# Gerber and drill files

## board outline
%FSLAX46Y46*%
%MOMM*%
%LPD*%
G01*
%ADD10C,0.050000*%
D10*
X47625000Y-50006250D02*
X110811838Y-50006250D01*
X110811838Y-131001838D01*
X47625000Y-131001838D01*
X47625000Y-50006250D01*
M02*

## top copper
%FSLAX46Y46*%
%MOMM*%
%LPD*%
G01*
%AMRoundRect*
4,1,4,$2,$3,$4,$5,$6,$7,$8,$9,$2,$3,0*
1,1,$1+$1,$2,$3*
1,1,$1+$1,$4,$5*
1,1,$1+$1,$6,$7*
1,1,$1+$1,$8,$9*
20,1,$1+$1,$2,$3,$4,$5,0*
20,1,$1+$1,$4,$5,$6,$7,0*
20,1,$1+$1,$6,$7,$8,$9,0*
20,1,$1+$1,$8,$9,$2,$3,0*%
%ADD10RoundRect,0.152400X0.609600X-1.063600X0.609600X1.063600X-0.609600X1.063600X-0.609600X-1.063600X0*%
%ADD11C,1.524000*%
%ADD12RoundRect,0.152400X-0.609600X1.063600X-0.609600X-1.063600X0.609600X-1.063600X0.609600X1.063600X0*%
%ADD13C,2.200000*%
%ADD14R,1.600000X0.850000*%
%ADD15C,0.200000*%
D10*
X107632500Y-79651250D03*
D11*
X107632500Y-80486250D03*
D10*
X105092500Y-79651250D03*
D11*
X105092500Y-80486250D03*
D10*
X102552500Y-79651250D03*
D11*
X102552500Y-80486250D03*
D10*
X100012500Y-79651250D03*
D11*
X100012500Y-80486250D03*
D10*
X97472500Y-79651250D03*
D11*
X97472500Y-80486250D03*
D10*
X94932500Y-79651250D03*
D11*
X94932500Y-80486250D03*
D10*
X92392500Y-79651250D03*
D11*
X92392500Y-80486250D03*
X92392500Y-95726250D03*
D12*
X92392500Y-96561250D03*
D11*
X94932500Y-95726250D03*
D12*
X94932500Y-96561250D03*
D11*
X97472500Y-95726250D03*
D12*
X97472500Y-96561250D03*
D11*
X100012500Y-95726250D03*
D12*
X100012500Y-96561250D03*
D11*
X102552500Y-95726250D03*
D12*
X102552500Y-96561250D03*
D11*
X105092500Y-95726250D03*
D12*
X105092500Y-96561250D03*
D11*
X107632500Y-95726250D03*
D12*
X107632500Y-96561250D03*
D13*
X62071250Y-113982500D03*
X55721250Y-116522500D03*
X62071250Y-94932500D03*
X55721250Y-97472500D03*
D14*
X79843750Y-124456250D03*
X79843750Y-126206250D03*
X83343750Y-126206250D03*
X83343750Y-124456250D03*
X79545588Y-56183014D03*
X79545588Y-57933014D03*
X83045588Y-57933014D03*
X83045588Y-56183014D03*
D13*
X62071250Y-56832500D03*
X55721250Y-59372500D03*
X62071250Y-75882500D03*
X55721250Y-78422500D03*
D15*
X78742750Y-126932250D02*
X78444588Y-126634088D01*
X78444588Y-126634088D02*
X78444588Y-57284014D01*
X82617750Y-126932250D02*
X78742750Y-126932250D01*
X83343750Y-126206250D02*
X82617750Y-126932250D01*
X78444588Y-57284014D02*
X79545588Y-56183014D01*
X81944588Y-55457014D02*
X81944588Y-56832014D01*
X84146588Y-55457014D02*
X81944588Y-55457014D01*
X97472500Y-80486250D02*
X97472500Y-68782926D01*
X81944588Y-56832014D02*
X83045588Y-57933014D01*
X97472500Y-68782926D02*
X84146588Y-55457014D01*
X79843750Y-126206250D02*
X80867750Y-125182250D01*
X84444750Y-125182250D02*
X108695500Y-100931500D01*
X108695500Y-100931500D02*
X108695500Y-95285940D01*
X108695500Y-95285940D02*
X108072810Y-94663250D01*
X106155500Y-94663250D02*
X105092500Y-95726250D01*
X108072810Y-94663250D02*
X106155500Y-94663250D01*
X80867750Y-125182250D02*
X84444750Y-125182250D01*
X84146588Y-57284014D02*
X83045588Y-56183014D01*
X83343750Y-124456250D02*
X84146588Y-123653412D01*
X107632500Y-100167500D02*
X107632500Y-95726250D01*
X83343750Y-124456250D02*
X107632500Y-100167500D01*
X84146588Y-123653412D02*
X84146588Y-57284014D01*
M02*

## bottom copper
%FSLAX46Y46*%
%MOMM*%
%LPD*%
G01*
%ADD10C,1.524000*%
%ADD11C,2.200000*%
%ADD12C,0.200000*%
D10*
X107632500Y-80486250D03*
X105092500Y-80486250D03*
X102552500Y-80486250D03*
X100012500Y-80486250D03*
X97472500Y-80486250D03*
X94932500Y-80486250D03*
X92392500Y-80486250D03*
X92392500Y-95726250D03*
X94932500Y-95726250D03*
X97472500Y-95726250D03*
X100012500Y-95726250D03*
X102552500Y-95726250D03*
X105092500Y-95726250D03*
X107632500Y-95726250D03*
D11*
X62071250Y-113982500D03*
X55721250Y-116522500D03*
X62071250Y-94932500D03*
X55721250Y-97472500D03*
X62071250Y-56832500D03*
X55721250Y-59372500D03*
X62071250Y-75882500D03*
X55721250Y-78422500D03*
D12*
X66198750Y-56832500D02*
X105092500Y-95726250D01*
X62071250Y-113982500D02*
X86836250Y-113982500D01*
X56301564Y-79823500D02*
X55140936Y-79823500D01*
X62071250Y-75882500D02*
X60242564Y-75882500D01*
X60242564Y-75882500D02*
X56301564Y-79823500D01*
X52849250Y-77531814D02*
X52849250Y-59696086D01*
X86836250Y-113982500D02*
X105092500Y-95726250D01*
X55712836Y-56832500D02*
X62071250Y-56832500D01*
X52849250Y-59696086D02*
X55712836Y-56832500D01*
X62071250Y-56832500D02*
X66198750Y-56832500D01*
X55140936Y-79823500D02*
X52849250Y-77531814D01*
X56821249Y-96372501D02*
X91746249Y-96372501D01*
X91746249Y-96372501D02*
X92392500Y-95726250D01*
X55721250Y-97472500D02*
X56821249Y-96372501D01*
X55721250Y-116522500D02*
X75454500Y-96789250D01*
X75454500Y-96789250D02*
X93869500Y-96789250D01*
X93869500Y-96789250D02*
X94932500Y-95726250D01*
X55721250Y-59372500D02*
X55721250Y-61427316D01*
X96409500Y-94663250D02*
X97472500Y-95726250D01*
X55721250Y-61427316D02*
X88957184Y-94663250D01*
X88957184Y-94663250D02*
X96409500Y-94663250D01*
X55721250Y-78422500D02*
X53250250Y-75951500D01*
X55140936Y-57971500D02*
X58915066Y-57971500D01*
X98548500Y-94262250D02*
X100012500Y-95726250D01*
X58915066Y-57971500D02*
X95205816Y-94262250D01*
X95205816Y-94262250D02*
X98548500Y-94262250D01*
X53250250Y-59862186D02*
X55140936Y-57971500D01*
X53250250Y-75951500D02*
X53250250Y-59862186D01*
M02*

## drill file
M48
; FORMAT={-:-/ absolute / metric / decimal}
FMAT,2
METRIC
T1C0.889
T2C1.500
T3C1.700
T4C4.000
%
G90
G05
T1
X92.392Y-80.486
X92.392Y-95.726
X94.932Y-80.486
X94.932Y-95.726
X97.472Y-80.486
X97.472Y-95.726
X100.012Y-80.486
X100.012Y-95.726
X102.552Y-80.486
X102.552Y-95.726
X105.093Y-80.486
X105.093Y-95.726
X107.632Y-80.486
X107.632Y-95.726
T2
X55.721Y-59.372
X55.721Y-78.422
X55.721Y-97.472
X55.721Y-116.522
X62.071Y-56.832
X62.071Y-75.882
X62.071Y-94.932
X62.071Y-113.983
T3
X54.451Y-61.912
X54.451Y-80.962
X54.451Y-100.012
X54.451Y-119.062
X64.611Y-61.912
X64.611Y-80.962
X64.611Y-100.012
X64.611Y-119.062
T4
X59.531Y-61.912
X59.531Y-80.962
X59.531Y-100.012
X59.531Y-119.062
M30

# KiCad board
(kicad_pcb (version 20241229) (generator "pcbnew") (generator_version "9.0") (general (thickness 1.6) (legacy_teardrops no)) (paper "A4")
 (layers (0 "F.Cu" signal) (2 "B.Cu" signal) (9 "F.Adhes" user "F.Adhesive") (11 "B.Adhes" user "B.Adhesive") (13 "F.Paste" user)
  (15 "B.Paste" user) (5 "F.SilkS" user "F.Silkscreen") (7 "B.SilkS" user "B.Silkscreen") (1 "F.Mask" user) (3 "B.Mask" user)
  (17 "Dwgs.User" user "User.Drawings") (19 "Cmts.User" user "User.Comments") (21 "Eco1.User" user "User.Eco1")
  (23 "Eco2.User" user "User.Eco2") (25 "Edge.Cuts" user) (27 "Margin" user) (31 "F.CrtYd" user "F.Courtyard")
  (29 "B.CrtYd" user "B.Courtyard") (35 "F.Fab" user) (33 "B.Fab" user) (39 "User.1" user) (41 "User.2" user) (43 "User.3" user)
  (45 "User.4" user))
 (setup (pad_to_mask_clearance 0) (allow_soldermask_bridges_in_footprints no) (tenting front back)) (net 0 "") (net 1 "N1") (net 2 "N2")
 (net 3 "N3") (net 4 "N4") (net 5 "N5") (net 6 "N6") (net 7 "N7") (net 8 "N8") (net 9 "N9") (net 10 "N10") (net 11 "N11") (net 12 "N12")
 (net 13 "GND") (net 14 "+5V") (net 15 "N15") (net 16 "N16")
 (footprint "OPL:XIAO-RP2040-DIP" (layer "F.Cu") (at 100.0125 88.10625 -90)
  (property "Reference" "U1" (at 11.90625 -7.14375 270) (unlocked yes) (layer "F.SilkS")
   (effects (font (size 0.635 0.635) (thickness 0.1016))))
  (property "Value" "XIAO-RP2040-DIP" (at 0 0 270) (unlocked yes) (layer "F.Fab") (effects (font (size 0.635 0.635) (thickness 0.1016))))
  (pad "1" smd roundrect (at -8.455 -7.62 90) (size 2.432 1.524) (layers "F.Cu" "F.Mask") (roundrect_rratio 0.1) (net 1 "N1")
   (thermal_bridge_angle 45))
  (pad "1" thru_hole circle (at -7.62 -7.62 90) (size 1.524 1.524) (drill 0.889) (layers "*.Cu" "*.Mask") (remove_unused_layers no)
   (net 1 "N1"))
  (pad "2" smd roundrect (at -8.455 -5.08 90) (size 2.432 1.524) (layers "F.Cu" "F.Mask") (roundrect_rratio 0.1) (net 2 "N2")
   (thermal_bridge_angle 45))
  (pad "2" thru_hole circle (at -7.62 -5.08 90) (size 1.524 1.524) (drill 0.889) (layers "*.Cu" "*.Mask") (remove_unused_layers no)
   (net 2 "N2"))
  (pad "3" smd roundrect (at -8.455 -2.54 90) (size 2.432 1.524) (layers "F.Cu" "F.Mask") (roundrect_rratio 0.1) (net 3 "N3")
   (thermal_bridge_angle 45))
  (pad "3" thru_hole circle (at -7.62 -2.54 90) (size 1.524 1.524) (drill 0.889) (layers "*.Cu" "*.Mask") (remove_unused_layers no)
   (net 3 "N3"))
  (pad "4" smd roundrect (at -8.455 0 90) (size 2.432 1.524) (layers "F.Cu" "F.Mask") (roundrect_rratio 0.1) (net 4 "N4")
   (thermal_bridge_angle 45))
  (pad "4" thru_hole circle (at -7.62 0 90) (size 1.524 1.524) (drill 0.889) (layers "*.Cu" "*.Mask") (remove_unused_layers no) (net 4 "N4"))
  (pad "5" smd roundrect (at -8.455 2.54 90) (size 2.432 1.524) (layers "F.Cu" "F.Mask") (roundrect_rratio 0.1) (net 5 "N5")
   (thermal_bridge_angle 45))
  (pad "5" thru_hole circle (at -7.62 2.54 90) (size 1.524 1.524) (drill 0.889) (layers "*.Cu" "*.Mask") (remove_unused_layers no)
   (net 5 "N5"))
  (pad "6" smd roundrect (at -8.455 5.08 90) (size 2.432 1.524) (layers "F.Cu" "F.Mask") (roundrect_rratio 0.1) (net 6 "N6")
   (thermal_bridge_angle 45))
  (pad "6" thru_hole circle (at -7.62 5.08 90) (size 1.524 1.524) (drill 0.889) (layers "*.Cu" "*.Mask") (remove_unused_layers no)
   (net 6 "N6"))
  (pad "7" smd roundrect (at -8.455 7.62 90) (size 2.432 1.524) (layers "F.Cu" "F.Mask") (roundrect_rratio 0.1) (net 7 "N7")
   (thermal_bridge_angle 45))
  (pad "7" thru_hole circle (at -7.62 7.62 90) (size 1.524 1.524) (drill 0.889) (layers "*.Cu" "*.Mask") (remove_unused_layers no)
   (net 7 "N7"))
  (pad "8" thru_hole circle (at 7.62 7.62 270) (size 1.524 1.524) (drill 0.889) (layers "*.Cu" "*.Mask") (remove_unused_layers no)
   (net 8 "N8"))
  (pad "8" smd roundrect (at 8.455 7.62 270) (size 2.432 1.524) (layers "F.Cu" "F.Mask") (roundrect_rratio 0.1) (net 8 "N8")
   (thermal_bridge_angle 45))
  (pad "9" thru_hole circle (at 7.62 5.08 270) (size 1.524 1.524) (drill 0.889) (layers "*.Cu" "*.Mask") (remove_unused_layers no)
   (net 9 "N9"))
  (pad "9" smd roundrect (at 8.455 5.08 270) (size 2.432 1.524) (layers "F.Cu" "F.Mask") (roundrect_rratio 0.1) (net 9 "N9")
   (thermal_bridge_angle 45))
  (pad "10" thru_hole circle (at 7.62 2.54 270) (size 1.524 1.524) (drill 0.889) (layers "*.Cu" "*.Mask") (remove_unused_layers no)
   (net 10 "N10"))
  (pad "10" smd roundrect (at 8.455 2.54 270) (size 2.432 1.524) (layers "F.Cu" "F.Mask") (roundrect_rratio 0.1) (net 10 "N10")
   (thermal_bridge_angle 45))
  (pad "11" thru_hole circle (at 7.62 0 270) (size 1.524 1.524) (drill 0.889) (layers "*.Cu" "*.Mask") (remove_unused_layers no)
   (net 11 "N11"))
  (pad "11" smd roundrect (at 8.455 0 270) (size 2.432 1.524) (layers "F.Cu" "F.Mask") (roundrect_rratio 0.1) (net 11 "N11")
   (thermal_bridge_angle 45))
  (pad "12" thru_hole circle (at 7.62 -2.54 270) (size 1.524 1.524) (drill 0.889) (layers "*.Cu" "*.Mask") (remove_unused_layers no)
   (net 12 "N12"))
  (pad "12" smd roundrect (at 8.455 -2.54 270) (size 2.432 1.524) (layers "F.Cu" "F.Mask") (roundrect_rratio 0.1) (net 12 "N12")
   (thermal_bridge_angle 45))
  (pad "13" thru_hole circle (at 7.62 -5.08 270) (size 1.524 1.524) (drill 0.889) (layers "*.Cu" "*.Mask") (remove_unused_layers no)
   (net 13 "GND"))
  (pad "13" smd roundrect (at 8.455 -5.08 270) (size 2.432 1.524) (layers "F.Cu" "F.Mask") (roundrect_rratio 0.1) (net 13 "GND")
   (thermal_bridge_angle 45))
  (pad "14" thru_hole circle (at 7.62 -7.62 270) (size 1.524 1.524) (drill 0.889) (layers "*.Cu" "*.Mask") (remove_unused_layers no)
   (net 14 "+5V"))
  (pad "14" smd roundrect (at 8.455 -7.62 270) (size 2.432 1.524) (layers "F.Cu" "F.Mask") (roundrect_rratio 0.1) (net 14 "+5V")
   (thermal_bridge_angle 45)))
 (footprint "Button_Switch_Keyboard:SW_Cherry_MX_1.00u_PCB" (layer "F.Cu") (at 62.07125 113.9825)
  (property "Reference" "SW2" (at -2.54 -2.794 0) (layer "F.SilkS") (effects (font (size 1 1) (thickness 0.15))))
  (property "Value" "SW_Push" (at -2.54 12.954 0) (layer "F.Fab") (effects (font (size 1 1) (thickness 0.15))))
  (pad "" np_thru_hole circle (at -7.62 5.08) (size 1.7 1.7) (drill 1.7) (layers "*.Cu" "*.Mask"))
  (pad "" np_thru_hole circle (at -2.54 5.08) (size 4 4) (drill 4) (layers "*.Cu" "*.Mask"))
  (pad "" np_thru_hole circle (at 2.54 5.08) (size 1.7 1.7) (drill 1.7) (layers "*.Cu" "*.Mask"))
  (pad "1" thru_hole circle (at 0 0) (size 2.2 2.2) (drill 1.5) (layers "*.Cu" "*.Mask") (remove_unused_layers no) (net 13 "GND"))
  (pad "2" thru_hole circle (at -6.35 2.54) (size 2.2 2.2) (drill 1.5) (layers "*.Cu" "*.Mask") (remove_unused_layers no) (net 9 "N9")))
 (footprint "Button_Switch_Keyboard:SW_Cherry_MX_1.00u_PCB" (layer "F.Cu") (at 62.07125 94.9325)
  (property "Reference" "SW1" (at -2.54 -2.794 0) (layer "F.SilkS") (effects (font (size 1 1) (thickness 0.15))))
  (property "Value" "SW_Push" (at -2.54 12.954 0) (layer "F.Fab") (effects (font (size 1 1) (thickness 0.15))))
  (pad "" np_thru_hole circle (at -7.62 5.08) (size 1.7 1.7) (drill 1.7) (layers "*.Cu" "*.Mask"))
  (pad "" np_thru_hole circle (at -2.54 5.08) (size 4 4) (drill 4) (layers "*.Cu" "*.Mask"))
  (pad "" np_thru_hole circle (at 2.54 5.08) (size 1.7 1.7) (drill 1.7) (layers "*.Cu" "*.Mask"))
  (pad "1" thru_hole circle (at 0 0) (size 2.2 2.2) (drill 1.5) (layers "*.Cu" "*.Mask") (remove_unused_layers no) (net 13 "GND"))
  (pad "2" thru_hole circle (at -6.35 2.54) (size 2.2 2.2) (drill 1.5) (layers "*.Cu" "*.Mask") (remove_unused_layers no) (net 8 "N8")))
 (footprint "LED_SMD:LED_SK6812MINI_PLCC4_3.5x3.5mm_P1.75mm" (layer "F.Cu") (at 81.59375 125.33125)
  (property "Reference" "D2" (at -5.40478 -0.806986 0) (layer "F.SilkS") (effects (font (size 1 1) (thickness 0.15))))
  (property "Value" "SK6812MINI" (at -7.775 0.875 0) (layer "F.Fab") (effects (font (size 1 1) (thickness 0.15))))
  (pad "1" smd rect (at -1.75 -0.875) (size 1.6 0.85) (layers "F.Cu" "F.Mask" "F.Paste") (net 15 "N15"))
  (pad "2" smd rect (at -1.75 0.875) (size 1.6 0.85) (layers "F.Cu" "F.Mask" "F.Paste") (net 13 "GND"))
  (pad "3" smd rect (at 1.75 0.875) (size 1.6 0.85) (layers "F.Cu" "F.Mask" "F.Paste") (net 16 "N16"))
  (pad "4" smd rect (at 1.75 -0.875) (size 1.6 0.85) (layers "F.Cu" "F.Mask" "F.Paste") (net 14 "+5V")))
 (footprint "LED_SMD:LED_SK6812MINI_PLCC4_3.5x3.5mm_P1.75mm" (layer "F.Cu") (at 81.295588 57.058014)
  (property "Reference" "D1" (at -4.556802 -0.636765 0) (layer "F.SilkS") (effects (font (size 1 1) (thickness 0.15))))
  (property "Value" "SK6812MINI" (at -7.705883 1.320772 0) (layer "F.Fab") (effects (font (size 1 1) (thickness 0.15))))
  (pad "1" smd rect (at -1.75 -0.875) (size 1.6 0.85) (layers "F.Cu" "F.Mask" "F.Paste") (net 16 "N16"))
  (pad "2" smd rect (at -1.75 0.875) (size 1.6 0.85) (layers "F.Cu" "F.Mask" "F.Paste") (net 13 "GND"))
  (pad "3" smd rect (at 1.75 0.875) (size 1.6 0.85) (layers "F.Cu" "F.Mask" "F.Paste") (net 5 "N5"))
  (pad "4" smd rect (at 1.75 -0.875) (size 1.6 0.85) (layers "F.Cu" "F.Mask" "F.Paste") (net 14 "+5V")))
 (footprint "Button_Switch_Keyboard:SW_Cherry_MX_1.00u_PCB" (layer "F.Cu") (at 62.07125 56.8325)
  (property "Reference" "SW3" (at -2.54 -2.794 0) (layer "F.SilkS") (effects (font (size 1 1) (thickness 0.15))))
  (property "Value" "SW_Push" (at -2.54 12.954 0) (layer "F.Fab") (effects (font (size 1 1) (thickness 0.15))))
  (pad "" np_thru_hole circle (at -7.62 5.08) (size 1.7 1.7) (drill 1.7) (layers "*.Cu" "*.Mask"))
  (pad "" np_thru_hole circle (at -2.54 5.08) (size 4 4) (drill 4) (layers "*.Cu" "*.Mask"))
  (pad "" np_thru_hole circle (at 2.54 5.08) (size 1.7 1.7) (drill 1.7) (layers "*.Cu" "*.Mask"))
  (pad "1" thru_hole circle (at 0 0) (size 2.2 2.2) (drill 1.5) (layers "*.Cu" "*.Mask") (remove_unused_layers no) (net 13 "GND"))
  (pad "2" thru_hole circle (at -6.35 2.54) (size 2.2 2.2) (drill 1.5) (layers "*.Cu" "*.Mask") (remove_unused_layers no) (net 10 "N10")))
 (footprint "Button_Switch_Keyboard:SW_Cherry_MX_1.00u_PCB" (layer "F.Cu") (at 62.07125 75.8825)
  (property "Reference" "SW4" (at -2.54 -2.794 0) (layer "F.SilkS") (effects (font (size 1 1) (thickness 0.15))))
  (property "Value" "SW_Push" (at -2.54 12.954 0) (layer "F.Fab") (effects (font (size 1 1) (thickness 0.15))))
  (pad "" np_thru_hole circle (at -7.62 5.08) (size 1.7 1.7) (drill 1.7) (layers "*.Cu" "*.Mask"))
  (pad "" np_thru_hole circle (at -2.54 5.08) (size 4 4) (drill 4) (layers "*.Cu" "*.Mask"))
  (pad "" np_thru_hole circle (at 2.54 5.08) (size 1.7 1.7) (drill 1.7) (layers "*.Cu" "*.Mask"))
  (pad "1" thru_hole circle (at 0 0) (size 2.2 2.2) (drill 1.5) (layers "*.Cu" "*.Mask") (remove_unused_layers no) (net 13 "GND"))
  (pad "2" thru_hole circle (at -6.35 2.54) (size 2.2 2.2) (drill 1.5) (layers "*.Cu" "*.Mask") (remove_unused_layers no) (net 11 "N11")))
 (gr_rect (start 47.625 50.00625) (end 110.811838 131.001838) (stroke (width 0.05) (type default)) (fill no) (layer "Edge.Cuts"))
 (segment (start 78.74275 126.93225) (end 78.444588 126.634088) (width 0.2) (layer "F.Cu") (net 16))
 (segment (start 78.444588 126.634088) (end 78.444588 57.284014) (width 0.2) (layer "F.Cu") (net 16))
 (segment (start 82.61775 126.93225) (end 78.74275 126.93225) (width 0.2) (layer "F.Cu") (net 16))
 (segment (start 83.34375 126.20625) (end 82.61775 126.93225) (width 0.2) (layer "F.Cu") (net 16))
 (segment (start 78.444588 57.284014) (end 79.545588 56.183014) (width 0.2) (layer "F.Cu") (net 16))
 (segment (start 81.944588 55.457014) (end 81.944588 56.832014) (width 0.2) (layer "F.Cu") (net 5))
 (segment (start 84.146588 55.457014) (end 81.944588 55.457014) (width 0.2) (layer "F.Cu") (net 5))
 (segment (start 97.4725 80.48625) (end 97.4725 68.782926) (width 0.2) (layer "F.Cu") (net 5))
 (segment (start 81.944588 56.832014) (end 83.045588 57.933014) (width 0.2) (layer "F.Cu") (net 5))
 (segment (start 97.4725 68.782926) (end 84.146588 55.457014) (width 0.2) (layer "F.Cu") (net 5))
 (segment (start 79.84375 126.20625) (end 80.86775 125.18225) (width 0.2) (layer "F.Cu") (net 13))
 (segment (start 84.44475 125.18225) (end 108.6955 100.9315) (width 0.2) (layer "F.Cu") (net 13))
 (segment (start 108.6955 100.9315) (end 108.6955 95.28594) (width 0.2) (layer "F.Cu") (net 13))
 (segment (start 108.6955 95.28594) (end 108.07281 94.66325) (width 0.2) (layer "F.Cu") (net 13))
 (segment (start 106.1555 94.66325) (end 105.0925 95.72625) (width 0.2) (layer "F.Cu") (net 13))
 (segment (start 108.07281 94.66325) (end 106.1555 94.66325) (width 0.2) (layer "F.Cu") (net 13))
 (segment (start 80.86775 125.18225) (end 84.44475 125.18225) (width 0.2) (layer "F.Cu") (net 13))
 (segment (start 66.19875 56.8325) (end 105.0925 95.72625) (width 0.2) (layer "B.Cu") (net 13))
 (segment (start 62.07125 113.9825) (end 86.83625 113.9825) (width 0.2) (layer "B.Cu") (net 13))
 (segment (start 56.301564 79.8235) (end 55.140936 79.8235) (width 0.2) (layer "B.Cu") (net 13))
 (segment (start 62.07125 75.8825) (end 60.242564 75.8825) (width 0.2) (layer "B.Cu") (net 13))
 (segment (start 60.242564 75.8825) (end 56.301564 79.8235) (width 0.2) (layer "B.Cu") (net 13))
 (segment (start 52.84925 77.531814) (end 52.84925 59.696086) (width 0.2) (layer "B.Cu") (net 13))
 (segment (start 86.83625 113.9825) (end 105.0925 95.72625) (width 0.2) (layer "B.Cu") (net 13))
 (segment (start 55.712836 56.8325) (end 62.07125 56.8325) (width 0.2) (layer "B.Cu") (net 13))
 (segment (start 52.84925 59.696086) (end 55.712836 56.8325) (width 0.2) (layer "B.Cu") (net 13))
 (segment (start 62.07125 56.8325) (end 66.19875 56.8325) (width 0.2) (layer "B.Cu") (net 13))
 (segment (start 55.140936 79.8235) (end 52.84925 77.531814) (width 0.2) (layer "B.Cu") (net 13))
 (segment (start 84.146588 57.284014) (end 83.045588 56.183014) (width 0.2) (layer "F.Cu") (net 14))
 (segment (start 83.34375 124.45625) (end 84.146588 123.653412) (width 0.2) (layer "F.Cu") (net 14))
 (segment (start 107.6325 100.1675) (end 107.6325 95.72625) (width 0.2) (layer "F.Cu") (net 14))
 (segment (start 83.34375 124.45625) (end 107.6325 100.1675) (width 0.2) (layer "F.Cu") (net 14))
 (segment (start 84.146588 123.653412) (end 84.146588 57.284014) (width 0.2) (layer "F.Cu") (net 14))
 (segment (start 56.821249 96.372501) (end 91.746249 96.372501) (width 0.2) (layer "B.Cu") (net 8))
 (segment (start 91.746249 96.372501) (end 92.3925 95.72625) (width 0.2) (layer "B.Cu") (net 8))
 (segment (start 55.72125 97.4725) (end 56.821249 96.372501) (width 0.2) (layer "B.Cu") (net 8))
 (segment (start 55.72125 116.5225) (end 75.4545 96.78925) (width 0.2) (layer "B.Cu") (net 9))
 (segment (start 75.4545 96.78925) (end 93.8695 96.78925) (width 0.2) (layer "B.Cu") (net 9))
 (segment (start 93.8695 96.78925) (end 94.9325 95.72625) (width 0.2) (layer "B.Cu") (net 9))
 (segment (start 55.72125 59.3725) (end 55.72125 61.427316) (width 0.2) (layer "B.Cu") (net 10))
 (segment (start 96.4095 94.66325) (end 97.4725 95.72625) (width 0.2) (layer "B.Cu") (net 10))
 (segment (start 55.72125 61.427316) (end 88.957184 94.66325) (width 0.2) (layer "B.Cu") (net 10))
 (segment (start 88.957184 94.66325) (end 96.4095 94.66325) (width 0.2) (layer "B.Cu") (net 10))
 (segment (start 55.72125 78.4225) (end 53.25025 75.9515) (width 0.2) (layer "B.Cu") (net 11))
 (segment (start 55.140936 57.9715) (end 58.915066 57.9715) (width 0.2) (layer "B.Cu") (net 11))
 (segment (start 98.5485 94.26225) (end 100.0125 95.72625) (width 0.2) (layer "B.Cu") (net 11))
 (segment (start 58.915066 57.9715) (end 95.205816 94.26225) (width 0.2) (layer "B.Cu") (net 11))
 (segment (start 95.205816 94.26225) (end 98.5485 94.26225) (width 0.2) (layer "B.Cu") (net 11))
 (segment (start 53.25025 59.862186) (end 55.140936 57.9715) (width 0.2) (layer "B.Cu") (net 11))
 (segment (start 53.25025 75.9515) (end 53.25025 59.862186) (width 0.2) (layer "B.Cu") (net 11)))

